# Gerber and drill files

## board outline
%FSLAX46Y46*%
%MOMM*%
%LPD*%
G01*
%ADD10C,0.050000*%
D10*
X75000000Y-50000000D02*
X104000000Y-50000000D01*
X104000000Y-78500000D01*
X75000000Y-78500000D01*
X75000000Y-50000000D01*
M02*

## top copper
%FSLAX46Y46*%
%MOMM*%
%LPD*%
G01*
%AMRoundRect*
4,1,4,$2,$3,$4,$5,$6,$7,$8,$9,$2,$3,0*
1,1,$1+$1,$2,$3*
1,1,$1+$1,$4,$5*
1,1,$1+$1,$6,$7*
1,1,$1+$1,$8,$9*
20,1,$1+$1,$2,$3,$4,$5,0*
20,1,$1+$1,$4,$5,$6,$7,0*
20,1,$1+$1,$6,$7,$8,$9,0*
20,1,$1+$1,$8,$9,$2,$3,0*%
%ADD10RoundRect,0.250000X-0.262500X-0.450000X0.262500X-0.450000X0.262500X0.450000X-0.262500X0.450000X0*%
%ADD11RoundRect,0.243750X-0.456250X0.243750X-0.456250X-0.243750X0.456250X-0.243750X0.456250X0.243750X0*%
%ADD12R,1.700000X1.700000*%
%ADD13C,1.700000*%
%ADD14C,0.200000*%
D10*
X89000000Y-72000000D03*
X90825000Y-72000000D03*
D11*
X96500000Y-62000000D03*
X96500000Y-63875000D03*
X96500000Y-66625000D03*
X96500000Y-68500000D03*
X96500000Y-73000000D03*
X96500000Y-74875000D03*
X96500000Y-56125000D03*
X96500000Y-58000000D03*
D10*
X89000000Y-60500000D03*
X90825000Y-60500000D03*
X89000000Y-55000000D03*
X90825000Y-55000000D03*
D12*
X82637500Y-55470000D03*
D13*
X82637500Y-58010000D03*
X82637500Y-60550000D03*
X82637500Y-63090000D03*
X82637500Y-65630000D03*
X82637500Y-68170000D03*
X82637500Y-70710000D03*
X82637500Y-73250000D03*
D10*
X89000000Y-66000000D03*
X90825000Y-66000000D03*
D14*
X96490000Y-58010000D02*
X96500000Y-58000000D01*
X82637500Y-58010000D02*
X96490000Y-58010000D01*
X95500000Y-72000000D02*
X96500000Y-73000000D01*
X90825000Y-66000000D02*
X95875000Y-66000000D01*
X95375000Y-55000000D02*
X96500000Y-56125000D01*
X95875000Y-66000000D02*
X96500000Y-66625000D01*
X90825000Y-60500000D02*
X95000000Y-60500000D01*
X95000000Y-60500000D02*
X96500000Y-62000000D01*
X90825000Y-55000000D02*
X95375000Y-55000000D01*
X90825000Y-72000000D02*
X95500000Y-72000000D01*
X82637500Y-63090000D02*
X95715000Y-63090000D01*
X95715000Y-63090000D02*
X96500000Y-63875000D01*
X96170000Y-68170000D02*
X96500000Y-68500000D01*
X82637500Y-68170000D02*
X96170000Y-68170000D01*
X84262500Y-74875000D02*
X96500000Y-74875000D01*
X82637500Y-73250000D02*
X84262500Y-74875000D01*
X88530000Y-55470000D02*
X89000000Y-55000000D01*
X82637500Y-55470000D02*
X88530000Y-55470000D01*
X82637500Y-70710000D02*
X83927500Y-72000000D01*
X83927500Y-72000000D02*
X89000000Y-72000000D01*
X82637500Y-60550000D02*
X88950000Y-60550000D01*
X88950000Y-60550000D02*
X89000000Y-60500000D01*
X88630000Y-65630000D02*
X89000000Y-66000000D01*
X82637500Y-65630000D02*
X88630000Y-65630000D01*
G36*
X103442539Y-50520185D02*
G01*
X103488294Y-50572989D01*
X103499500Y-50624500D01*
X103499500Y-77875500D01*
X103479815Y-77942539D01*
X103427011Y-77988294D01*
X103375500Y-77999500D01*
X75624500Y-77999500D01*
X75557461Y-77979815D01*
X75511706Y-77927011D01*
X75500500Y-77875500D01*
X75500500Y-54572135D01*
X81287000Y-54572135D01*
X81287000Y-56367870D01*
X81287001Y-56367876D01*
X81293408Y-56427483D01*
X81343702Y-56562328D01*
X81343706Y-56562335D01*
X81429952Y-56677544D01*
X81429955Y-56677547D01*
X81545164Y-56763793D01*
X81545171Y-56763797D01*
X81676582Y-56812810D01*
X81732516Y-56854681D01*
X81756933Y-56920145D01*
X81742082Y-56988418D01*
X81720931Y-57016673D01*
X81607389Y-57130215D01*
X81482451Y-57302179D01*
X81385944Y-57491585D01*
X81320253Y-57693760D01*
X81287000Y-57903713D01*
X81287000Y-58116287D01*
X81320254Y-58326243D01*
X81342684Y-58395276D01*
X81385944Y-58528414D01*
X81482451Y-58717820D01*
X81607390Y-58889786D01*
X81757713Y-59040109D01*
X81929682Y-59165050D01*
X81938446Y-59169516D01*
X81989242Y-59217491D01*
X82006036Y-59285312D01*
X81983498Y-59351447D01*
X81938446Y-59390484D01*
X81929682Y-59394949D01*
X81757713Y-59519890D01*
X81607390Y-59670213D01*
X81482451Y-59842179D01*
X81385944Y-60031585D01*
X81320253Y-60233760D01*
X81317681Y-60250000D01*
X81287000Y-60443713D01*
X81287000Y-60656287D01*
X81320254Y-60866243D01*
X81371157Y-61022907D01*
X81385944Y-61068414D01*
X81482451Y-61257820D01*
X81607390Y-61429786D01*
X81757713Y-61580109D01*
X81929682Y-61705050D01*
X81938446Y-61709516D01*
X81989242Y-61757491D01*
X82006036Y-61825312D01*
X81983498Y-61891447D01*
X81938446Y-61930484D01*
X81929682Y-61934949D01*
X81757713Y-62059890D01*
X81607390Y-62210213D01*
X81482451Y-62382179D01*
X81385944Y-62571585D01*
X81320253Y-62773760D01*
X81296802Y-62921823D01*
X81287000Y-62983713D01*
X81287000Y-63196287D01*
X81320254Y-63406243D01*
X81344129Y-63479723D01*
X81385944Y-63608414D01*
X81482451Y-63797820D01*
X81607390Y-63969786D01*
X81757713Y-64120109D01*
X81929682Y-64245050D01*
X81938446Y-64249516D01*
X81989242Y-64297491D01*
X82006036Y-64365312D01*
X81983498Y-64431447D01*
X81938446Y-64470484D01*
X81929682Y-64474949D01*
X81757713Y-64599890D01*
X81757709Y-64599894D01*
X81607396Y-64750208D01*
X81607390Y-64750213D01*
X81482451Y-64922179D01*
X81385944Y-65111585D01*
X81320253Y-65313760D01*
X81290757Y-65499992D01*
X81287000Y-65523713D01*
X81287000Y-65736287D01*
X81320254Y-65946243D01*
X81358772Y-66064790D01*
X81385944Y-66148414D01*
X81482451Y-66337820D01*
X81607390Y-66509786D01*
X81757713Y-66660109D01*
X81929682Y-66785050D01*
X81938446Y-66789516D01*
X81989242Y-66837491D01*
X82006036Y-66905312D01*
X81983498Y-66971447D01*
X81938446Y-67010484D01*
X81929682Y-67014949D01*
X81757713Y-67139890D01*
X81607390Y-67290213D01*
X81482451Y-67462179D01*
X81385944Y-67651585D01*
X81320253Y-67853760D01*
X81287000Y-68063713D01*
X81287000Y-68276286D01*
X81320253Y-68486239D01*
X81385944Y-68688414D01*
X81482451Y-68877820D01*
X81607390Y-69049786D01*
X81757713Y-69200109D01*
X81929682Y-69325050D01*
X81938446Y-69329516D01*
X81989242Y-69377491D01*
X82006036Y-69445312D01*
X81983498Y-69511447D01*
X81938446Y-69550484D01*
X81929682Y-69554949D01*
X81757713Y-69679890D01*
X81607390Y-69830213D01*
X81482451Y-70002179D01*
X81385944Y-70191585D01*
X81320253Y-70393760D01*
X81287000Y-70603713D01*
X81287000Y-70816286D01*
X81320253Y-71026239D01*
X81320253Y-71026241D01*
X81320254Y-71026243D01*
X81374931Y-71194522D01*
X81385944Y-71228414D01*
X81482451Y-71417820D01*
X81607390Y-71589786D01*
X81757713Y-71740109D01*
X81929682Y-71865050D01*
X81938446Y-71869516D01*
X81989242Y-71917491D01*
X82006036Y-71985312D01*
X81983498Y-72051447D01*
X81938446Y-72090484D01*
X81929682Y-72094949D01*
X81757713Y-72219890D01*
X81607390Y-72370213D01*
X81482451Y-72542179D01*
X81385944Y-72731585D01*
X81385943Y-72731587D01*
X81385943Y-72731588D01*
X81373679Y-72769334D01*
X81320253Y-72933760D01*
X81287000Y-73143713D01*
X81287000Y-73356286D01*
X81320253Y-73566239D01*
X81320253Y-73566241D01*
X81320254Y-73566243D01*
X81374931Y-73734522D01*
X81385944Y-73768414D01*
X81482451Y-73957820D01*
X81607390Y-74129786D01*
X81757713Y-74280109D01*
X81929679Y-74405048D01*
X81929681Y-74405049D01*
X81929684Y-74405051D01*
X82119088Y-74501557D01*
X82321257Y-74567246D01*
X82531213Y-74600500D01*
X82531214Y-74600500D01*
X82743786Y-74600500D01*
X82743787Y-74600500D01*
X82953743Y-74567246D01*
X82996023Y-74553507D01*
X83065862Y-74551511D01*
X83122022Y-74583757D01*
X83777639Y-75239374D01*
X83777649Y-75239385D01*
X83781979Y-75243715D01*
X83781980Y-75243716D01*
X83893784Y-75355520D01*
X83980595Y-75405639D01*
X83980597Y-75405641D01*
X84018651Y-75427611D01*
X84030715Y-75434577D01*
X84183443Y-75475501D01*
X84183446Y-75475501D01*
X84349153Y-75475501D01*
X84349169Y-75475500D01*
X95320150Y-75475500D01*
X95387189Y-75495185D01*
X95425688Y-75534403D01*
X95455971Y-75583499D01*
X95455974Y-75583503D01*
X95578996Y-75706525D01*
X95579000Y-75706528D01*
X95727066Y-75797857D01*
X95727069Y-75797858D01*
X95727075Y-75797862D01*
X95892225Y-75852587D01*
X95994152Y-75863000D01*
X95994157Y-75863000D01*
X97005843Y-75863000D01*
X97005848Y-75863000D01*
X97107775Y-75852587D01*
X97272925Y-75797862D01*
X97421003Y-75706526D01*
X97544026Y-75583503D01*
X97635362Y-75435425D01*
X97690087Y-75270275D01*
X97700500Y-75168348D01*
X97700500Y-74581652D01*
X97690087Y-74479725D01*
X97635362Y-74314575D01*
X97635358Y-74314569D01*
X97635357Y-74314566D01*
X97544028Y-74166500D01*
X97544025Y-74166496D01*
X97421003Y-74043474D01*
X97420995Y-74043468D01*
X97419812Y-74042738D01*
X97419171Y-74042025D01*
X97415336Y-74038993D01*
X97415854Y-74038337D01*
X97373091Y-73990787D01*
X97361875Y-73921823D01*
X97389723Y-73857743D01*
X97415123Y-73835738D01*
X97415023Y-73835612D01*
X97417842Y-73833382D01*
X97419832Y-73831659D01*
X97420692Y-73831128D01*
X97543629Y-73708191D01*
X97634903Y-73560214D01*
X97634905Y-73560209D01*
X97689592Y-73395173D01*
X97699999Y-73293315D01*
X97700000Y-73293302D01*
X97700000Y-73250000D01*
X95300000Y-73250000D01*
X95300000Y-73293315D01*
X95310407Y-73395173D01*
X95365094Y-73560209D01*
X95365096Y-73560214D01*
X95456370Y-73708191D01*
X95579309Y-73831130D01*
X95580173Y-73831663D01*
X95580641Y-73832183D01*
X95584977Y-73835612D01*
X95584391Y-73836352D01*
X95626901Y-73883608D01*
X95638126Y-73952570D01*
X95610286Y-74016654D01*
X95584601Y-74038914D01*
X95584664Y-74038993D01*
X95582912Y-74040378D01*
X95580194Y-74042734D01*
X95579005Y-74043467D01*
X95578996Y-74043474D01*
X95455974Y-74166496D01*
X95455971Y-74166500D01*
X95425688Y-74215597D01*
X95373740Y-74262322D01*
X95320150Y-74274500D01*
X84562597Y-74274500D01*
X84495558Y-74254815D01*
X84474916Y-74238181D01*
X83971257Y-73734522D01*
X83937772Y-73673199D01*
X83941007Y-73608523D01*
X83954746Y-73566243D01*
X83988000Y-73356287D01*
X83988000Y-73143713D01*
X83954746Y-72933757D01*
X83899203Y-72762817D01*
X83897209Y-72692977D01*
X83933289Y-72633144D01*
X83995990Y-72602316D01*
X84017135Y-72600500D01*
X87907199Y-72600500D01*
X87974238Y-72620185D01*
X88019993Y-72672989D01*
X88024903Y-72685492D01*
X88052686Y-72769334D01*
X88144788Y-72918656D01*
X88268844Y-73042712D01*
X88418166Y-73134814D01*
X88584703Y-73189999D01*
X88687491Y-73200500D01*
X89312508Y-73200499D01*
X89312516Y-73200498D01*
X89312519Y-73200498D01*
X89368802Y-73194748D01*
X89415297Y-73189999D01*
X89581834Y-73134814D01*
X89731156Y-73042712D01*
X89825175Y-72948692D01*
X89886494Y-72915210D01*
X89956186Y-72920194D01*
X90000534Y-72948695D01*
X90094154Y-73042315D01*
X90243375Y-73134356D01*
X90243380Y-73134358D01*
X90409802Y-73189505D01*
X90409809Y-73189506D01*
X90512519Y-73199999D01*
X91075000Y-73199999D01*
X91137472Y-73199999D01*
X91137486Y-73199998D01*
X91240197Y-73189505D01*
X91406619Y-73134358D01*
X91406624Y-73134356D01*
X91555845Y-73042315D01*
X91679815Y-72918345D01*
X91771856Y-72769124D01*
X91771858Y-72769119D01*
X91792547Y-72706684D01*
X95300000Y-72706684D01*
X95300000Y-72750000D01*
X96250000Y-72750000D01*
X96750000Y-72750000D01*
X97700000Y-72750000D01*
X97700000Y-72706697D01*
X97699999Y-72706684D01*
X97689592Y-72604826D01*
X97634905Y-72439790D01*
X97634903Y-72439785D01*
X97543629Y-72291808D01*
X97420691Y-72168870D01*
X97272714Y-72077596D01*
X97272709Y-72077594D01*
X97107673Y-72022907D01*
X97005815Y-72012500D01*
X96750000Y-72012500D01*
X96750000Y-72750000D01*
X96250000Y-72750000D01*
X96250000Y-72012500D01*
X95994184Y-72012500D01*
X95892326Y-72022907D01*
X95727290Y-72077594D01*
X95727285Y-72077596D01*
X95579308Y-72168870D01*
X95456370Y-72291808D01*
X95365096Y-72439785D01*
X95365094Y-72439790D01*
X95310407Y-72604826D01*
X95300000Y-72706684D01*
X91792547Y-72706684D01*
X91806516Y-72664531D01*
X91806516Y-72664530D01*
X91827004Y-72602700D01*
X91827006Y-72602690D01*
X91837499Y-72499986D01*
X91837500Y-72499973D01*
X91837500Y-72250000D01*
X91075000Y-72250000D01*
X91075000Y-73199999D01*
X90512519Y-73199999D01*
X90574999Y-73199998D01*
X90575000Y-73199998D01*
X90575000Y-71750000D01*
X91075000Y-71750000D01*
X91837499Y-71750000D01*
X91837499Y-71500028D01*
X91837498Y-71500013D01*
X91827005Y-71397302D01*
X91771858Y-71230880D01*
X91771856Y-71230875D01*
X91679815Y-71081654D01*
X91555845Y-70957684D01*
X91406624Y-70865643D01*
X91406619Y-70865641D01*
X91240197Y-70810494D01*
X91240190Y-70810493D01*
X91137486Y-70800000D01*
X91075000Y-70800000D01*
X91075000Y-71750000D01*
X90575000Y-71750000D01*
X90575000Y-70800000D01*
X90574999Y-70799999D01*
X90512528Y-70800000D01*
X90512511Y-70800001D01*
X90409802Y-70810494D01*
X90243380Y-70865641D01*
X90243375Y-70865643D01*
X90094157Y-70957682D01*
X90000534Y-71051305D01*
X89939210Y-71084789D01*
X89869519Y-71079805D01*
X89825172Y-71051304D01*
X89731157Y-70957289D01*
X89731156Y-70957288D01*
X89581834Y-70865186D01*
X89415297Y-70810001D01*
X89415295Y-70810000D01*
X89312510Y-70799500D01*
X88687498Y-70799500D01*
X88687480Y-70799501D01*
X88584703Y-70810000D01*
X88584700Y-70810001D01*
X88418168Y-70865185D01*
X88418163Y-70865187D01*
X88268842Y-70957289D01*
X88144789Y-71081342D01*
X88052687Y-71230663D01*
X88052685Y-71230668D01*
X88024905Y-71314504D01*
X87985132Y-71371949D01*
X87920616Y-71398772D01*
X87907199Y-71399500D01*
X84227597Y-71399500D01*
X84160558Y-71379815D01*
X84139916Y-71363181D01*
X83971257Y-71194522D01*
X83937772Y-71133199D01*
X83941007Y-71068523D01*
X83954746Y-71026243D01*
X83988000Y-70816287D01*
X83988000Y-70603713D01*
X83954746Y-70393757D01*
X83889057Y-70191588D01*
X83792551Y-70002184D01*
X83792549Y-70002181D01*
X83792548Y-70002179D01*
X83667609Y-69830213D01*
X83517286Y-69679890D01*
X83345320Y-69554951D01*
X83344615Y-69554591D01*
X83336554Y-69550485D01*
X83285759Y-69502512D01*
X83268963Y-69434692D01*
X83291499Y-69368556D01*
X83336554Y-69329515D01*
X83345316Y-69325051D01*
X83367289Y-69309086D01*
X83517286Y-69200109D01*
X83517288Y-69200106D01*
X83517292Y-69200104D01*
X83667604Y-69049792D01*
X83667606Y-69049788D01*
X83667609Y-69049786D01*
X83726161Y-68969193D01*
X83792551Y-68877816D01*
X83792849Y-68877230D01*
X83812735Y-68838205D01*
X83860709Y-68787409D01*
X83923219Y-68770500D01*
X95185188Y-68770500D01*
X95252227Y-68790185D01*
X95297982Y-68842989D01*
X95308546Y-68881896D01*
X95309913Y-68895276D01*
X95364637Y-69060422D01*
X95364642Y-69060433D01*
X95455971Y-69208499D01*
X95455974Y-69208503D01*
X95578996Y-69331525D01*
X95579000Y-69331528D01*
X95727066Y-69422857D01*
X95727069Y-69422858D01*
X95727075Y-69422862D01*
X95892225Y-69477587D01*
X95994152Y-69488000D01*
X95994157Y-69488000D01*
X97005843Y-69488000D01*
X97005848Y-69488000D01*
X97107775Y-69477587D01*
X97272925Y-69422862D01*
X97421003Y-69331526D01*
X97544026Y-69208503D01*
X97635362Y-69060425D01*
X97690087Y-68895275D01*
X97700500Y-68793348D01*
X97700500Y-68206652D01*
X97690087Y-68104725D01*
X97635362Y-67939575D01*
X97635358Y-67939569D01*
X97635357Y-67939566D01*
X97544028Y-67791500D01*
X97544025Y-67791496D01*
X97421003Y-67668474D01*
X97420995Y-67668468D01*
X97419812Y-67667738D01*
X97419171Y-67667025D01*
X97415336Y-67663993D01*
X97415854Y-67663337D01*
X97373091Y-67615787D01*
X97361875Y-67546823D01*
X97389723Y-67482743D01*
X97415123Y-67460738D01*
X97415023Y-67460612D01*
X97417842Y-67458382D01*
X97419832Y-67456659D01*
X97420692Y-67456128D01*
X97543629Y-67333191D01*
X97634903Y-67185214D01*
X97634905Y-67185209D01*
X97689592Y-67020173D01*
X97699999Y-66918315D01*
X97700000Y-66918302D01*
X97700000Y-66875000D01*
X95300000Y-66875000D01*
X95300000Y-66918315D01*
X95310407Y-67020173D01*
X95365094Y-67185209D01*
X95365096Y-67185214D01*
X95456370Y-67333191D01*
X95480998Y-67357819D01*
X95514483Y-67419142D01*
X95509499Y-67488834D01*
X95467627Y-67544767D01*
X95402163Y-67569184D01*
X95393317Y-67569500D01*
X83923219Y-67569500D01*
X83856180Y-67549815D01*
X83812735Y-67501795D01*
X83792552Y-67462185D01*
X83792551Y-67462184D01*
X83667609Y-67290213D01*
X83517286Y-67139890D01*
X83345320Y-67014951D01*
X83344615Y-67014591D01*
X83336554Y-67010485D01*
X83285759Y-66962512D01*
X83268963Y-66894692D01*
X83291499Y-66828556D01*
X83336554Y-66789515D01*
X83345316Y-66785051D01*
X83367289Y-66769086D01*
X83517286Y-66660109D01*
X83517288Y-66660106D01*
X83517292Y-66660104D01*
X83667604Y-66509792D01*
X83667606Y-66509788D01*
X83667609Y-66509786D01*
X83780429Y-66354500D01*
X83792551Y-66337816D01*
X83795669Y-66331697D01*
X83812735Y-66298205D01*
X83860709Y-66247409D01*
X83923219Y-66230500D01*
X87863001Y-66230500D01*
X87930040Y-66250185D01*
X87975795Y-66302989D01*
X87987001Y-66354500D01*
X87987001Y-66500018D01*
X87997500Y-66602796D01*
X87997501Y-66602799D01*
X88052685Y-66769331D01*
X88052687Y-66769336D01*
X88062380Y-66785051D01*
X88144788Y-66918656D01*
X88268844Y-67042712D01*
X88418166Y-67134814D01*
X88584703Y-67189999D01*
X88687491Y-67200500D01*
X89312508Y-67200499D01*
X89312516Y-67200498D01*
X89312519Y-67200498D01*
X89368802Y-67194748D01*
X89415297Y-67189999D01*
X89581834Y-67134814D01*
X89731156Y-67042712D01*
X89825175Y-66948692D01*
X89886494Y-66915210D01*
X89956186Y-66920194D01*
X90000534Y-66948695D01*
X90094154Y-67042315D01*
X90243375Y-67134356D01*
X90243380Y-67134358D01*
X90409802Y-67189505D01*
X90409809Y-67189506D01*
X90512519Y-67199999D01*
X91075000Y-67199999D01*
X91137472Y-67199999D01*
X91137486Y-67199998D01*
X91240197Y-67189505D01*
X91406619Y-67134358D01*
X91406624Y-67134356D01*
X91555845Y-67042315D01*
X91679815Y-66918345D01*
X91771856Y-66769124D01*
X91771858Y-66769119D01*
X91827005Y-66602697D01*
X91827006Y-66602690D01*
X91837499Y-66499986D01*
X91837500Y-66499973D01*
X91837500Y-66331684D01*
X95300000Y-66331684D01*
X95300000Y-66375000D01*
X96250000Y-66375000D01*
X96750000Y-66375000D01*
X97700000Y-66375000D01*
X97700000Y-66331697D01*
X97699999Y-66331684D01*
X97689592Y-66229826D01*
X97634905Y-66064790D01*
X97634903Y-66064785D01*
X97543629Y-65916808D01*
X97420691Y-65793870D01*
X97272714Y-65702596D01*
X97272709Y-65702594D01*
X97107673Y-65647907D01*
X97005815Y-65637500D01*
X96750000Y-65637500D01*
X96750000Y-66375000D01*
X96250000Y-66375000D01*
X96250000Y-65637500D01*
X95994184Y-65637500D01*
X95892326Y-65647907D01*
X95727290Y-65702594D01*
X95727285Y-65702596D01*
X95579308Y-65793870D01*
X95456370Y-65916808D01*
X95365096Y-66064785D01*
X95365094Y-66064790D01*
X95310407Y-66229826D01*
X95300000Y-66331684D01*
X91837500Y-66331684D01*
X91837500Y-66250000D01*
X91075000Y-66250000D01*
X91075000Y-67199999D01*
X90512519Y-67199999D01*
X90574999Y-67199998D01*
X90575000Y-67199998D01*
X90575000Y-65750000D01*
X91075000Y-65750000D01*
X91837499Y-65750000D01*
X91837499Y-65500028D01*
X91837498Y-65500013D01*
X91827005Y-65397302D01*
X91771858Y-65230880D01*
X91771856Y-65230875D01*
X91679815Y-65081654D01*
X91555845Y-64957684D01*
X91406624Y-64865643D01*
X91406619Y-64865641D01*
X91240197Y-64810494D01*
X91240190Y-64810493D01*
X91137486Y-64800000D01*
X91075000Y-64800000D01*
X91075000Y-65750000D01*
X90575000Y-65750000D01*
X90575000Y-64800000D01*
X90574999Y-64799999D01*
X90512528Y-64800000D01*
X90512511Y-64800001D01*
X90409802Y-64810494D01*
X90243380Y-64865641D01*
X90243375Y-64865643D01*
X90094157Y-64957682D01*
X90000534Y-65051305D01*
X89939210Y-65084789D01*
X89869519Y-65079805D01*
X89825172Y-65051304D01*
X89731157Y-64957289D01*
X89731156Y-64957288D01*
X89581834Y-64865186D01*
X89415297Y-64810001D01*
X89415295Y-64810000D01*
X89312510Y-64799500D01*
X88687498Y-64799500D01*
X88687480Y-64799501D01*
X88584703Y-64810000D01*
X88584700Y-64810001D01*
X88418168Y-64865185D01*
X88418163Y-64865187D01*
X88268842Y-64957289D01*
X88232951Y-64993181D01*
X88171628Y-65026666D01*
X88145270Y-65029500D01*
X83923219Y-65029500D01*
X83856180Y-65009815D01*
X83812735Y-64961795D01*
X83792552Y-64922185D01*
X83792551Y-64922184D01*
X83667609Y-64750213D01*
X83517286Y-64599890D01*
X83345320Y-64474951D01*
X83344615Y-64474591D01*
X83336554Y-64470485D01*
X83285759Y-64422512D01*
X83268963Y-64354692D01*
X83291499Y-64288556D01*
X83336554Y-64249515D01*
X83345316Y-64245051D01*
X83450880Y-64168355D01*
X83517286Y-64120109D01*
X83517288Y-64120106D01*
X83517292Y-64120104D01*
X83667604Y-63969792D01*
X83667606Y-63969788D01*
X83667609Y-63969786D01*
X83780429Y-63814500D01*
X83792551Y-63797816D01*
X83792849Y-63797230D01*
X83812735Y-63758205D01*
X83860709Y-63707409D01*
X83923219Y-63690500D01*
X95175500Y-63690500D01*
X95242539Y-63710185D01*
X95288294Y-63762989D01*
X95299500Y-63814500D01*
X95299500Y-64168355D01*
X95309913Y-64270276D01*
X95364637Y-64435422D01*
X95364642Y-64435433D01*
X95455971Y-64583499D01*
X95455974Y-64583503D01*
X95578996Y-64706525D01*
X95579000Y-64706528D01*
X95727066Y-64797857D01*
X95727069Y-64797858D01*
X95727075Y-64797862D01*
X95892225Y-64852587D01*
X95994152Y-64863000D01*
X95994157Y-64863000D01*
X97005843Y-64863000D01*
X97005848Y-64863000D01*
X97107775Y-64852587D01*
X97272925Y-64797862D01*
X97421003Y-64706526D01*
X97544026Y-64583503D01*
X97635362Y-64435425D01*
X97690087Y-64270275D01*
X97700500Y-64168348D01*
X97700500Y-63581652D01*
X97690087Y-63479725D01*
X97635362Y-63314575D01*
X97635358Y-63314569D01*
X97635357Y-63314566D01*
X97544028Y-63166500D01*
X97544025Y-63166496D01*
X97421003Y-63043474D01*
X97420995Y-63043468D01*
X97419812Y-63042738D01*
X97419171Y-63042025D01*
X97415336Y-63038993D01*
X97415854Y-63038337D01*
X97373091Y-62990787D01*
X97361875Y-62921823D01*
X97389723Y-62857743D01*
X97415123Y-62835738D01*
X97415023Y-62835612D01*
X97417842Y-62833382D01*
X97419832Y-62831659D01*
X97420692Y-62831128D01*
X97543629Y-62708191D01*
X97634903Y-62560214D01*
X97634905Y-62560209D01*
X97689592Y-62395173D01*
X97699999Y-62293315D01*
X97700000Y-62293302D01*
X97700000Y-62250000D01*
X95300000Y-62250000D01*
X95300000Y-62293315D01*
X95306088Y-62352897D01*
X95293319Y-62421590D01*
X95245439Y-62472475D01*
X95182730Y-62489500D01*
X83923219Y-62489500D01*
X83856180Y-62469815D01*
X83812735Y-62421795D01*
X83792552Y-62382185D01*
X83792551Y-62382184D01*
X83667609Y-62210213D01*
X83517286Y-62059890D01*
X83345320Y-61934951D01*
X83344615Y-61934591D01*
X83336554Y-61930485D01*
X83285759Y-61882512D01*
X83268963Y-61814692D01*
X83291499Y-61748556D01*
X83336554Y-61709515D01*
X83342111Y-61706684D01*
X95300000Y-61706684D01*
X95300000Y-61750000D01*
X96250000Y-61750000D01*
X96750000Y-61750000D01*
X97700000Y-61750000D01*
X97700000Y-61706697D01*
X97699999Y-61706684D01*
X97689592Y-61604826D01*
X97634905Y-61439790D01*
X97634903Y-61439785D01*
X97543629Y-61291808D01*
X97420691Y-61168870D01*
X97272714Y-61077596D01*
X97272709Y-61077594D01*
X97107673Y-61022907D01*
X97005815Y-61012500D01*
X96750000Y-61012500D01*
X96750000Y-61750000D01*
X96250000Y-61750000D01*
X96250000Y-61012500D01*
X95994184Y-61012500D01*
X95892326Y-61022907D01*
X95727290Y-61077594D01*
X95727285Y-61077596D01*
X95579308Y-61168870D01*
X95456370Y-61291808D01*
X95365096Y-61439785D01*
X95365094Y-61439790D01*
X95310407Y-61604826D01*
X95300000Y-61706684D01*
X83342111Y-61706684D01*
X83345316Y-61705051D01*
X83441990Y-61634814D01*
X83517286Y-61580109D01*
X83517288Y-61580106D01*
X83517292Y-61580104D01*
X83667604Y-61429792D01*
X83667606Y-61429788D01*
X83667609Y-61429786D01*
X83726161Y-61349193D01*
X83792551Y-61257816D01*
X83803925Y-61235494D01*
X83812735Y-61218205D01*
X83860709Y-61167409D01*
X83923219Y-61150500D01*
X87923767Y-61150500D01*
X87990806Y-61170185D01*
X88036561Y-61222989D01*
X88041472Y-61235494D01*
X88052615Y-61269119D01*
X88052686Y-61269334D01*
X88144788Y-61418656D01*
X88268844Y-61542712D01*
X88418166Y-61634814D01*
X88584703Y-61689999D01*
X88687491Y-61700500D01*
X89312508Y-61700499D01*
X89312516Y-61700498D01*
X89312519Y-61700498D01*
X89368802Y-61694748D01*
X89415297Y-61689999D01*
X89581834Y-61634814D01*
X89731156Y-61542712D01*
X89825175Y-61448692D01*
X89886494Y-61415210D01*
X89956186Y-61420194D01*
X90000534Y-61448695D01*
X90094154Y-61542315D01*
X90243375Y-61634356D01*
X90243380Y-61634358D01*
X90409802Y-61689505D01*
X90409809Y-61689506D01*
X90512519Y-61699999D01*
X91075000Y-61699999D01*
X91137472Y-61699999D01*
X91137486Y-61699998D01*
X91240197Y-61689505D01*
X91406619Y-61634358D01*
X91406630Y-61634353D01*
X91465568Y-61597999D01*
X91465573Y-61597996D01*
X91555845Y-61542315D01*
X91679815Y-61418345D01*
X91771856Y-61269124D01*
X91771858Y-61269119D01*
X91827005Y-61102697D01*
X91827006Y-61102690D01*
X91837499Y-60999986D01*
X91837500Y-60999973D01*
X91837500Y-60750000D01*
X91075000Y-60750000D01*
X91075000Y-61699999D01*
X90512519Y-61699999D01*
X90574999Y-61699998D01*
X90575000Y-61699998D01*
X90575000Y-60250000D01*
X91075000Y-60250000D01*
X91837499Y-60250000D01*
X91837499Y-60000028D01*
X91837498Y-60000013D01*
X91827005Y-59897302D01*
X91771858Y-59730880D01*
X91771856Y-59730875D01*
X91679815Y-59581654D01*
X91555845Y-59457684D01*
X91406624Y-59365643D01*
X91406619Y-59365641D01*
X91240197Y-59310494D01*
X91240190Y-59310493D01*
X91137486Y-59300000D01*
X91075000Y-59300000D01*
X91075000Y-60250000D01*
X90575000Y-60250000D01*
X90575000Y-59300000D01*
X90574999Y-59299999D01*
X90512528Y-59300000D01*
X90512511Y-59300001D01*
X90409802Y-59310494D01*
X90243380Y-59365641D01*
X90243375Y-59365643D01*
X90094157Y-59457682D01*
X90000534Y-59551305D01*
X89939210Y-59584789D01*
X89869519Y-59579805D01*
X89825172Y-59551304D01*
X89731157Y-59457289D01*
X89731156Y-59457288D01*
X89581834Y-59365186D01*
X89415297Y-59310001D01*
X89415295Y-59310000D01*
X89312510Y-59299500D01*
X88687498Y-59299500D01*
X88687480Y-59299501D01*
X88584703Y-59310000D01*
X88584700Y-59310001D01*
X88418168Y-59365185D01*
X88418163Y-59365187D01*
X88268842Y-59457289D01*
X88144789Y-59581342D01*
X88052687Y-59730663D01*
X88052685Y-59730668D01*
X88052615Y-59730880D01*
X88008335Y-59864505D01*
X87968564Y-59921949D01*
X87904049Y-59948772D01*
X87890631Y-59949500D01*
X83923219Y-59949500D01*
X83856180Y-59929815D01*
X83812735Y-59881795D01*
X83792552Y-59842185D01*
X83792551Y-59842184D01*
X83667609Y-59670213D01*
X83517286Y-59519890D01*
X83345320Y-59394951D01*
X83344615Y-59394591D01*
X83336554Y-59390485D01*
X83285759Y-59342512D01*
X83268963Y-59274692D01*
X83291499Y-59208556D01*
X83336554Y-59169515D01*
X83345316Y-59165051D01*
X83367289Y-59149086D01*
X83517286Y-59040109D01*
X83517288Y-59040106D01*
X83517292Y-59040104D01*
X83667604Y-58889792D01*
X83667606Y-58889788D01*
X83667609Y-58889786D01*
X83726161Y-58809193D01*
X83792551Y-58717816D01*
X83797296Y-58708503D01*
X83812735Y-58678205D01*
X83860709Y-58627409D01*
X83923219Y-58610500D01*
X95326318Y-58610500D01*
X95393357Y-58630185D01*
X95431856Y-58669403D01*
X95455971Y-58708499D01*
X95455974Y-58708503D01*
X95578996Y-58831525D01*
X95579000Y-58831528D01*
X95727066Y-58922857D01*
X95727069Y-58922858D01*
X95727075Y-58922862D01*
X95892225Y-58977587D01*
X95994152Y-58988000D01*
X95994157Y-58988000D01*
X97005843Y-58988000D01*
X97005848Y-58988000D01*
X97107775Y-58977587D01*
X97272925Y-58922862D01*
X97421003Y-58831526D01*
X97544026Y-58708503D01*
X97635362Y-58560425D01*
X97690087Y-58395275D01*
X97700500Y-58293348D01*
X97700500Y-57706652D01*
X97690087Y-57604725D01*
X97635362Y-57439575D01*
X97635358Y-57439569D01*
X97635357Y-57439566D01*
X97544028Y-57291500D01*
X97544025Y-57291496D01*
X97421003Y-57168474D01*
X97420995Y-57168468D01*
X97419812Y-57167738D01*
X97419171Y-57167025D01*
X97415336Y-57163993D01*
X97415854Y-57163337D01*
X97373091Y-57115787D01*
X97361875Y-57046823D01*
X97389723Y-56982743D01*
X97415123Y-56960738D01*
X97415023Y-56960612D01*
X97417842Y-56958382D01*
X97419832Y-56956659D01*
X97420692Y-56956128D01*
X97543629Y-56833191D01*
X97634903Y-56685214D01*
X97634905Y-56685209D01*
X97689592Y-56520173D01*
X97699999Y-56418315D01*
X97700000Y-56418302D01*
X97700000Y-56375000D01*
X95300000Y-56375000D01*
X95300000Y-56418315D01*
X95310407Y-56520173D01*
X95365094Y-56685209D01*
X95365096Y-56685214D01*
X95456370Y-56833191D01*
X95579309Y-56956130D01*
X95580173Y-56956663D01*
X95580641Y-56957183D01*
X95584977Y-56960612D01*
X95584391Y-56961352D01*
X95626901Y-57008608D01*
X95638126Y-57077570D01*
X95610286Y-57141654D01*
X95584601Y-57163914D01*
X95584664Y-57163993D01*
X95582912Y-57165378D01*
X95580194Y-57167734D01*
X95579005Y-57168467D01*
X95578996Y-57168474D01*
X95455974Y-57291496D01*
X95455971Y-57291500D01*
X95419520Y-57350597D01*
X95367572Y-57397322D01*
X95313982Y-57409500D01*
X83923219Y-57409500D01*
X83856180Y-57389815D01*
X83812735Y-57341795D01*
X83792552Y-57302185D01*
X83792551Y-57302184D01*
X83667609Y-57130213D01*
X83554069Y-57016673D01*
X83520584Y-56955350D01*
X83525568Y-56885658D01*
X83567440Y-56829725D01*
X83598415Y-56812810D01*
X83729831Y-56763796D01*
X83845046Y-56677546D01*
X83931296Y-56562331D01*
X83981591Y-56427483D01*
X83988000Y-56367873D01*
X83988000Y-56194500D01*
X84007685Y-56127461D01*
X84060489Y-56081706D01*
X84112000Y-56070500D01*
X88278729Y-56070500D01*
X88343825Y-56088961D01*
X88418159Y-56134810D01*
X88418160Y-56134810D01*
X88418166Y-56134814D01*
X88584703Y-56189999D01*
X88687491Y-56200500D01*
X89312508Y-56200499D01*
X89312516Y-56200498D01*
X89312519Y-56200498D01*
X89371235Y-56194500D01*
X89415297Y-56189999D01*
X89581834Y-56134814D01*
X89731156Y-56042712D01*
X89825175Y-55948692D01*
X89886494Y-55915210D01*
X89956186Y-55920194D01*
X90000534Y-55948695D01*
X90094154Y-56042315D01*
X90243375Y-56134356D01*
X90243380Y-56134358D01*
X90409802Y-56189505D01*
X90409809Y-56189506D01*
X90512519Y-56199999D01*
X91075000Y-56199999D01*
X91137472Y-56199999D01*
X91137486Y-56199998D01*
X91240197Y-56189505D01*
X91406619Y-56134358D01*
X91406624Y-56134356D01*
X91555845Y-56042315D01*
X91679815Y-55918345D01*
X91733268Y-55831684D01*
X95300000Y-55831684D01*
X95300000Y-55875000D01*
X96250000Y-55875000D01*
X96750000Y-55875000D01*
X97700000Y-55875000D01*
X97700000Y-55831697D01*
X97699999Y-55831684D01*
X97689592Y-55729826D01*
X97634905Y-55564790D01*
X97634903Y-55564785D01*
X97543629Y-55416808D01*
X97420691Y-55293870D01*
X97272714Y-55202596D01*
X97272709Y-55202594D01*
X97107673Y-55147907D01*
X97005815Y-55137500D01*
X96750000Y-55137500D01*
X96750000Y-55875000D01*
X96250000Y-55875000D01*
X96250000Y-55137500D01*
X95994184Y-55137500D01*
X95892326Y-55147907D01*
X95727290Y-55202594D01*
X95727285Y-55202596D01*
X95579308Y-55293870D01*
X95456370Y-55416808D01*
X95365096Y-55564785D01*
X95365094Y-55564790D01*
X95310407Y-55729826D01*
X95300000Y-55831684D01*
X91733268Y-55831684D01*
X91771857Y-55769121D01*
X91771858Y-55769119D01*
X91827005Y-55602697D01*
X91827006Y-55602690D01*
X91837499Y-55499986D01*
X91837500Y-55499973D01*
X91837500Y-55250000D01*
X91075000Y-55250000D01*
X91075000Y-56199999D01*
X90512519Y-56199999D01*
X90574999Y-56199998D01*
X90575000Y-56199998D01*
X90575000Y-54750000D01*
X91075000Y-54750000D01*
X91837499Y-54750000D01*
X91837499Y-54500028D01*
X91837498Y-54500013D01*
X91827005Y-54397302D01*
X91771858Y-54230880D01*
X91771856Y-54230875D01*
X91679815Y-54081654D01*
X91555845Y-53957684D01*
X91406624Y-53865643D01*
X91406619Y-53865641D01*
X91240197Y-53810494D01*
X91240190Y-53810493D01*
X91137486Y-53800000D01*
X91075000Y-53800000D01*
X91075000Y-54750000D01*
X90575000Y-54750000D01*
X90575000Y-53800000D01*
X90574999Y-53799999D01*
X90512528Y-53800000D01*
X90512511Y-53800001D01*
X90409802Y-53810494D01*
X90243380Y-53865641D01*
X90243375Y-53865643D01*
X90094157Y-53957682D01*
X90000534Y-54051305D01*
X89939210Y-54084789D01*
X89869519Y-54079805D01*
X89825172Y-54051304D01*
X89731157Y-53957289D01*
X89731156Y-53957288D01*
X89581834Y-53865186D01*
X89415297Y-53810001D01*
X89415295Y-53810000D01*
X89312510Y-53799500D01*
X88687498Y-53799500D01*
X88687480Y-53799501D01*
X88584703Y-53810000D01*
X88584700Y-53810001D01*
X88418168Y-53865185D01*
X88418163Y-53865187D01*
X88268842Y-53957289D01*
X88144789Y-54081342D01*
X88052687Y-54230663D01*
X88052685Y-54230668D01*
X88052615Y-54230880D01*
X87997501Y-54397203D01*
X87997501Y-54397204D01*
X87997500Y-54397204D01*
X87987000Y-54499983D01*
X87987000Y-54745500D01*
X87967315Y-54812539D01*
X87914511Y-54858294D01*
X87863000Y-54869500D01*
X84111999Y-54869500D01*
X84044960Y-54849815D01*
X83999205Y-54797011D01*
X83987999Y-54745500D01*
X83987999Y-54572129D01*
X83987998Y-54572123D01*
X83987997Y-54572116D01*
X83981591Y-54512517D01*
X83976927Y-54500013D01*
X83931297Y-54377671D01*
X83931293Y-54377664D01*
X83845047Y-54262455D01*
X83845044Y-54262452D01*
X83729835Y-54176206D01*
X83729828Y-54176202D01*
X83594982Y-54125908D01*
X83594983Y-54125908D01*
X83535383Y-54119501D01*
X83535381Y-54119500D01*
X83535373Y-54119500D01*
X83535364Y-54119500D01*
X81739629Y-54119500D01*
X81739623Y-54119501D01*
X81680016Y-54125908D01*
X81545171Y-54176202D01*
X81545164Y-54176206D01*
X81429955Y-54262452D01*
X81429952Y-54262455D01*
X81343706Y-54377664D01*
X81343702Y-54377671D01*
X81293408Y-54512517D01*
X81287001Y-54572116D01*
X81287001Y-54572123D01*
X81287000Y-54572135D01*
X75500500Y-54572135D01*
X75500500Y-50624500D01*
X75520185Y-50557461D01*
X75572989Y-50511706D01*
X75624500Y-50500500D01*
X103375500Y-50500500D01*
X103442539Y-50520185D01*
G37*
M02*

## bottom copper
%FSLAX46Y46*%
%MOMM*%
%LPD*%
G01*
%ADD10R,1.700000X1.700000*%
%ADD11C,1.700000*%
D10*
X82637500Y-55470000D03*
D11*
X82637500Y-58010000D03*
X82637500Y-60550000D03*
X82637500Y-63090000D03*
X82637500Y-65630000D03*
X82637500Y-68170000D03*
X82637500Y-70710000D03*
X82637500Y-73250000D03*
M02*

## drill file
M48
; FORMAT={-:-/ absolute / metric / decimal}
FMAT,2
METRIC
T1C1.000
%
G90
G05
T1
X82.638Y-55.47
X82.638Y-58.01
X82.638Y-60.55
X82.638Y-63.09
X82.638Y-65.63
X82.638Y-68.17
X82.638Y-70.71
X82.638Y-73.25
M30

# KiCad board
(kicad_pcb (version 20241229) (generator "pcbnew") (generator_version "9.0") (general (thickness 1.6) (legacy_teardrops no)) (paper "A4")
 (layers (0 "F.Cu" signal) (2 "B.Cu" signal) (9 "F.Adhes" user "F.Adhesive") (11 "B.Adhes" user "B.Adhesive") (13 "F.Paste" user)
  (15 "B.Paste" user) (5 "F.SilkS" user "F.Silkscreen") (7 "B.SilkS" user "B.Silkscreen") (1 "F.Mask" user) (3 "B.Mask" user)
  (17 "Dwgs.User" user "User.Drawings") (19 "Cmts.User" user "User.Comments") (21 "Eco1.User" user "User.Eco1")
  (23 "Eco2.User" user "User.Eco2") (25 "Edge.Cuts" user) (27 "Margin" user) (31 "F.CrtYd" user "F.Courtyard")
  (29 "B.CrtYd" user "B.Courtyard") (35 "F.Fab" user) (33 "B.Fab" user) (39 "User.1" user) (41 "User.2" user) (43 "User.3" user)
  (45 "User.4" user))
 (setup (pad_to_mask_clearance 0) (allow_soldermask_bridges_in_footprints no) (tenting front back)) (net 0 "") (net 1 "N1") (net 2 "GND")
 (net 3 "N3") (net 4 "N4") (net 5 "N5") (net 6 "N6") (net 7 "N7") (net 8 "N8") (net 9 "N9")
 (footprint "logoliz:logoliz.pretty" (layer "F.Cu") (at 101 53.5)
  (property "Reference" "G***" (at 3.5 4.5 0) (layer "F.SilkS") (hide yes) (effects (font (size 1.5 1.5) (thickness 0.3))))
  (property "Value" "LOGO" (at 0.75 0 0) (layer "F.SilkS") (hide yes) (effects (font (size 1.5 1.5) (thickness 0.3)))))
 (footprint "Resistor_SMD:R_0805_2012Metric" (layer "F.Cu") (at 89.9125 72)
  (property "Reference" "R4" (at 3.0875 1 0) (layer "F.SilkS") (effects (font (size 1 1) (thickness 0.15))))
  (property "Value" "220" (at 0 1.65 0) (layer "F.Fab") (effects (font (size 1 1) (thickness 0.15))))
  (pad "1" smd roundrect (at -0.9125 0) (size 1.025 1.4) (layers "F.Cu" "F.Mask" "F.Paste") (roundrect_rratio 0.243902) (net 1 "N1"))
  (pad "2" smd roundrect (at 0.9125 0) (size 1.025 1.4) (layers "F.Cu" "F.Mask" "F.Paste") (roundrect_rratio 0.243902) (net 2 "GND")))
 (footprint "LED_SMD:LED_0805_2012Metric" (layer "F.Cu") (at 96.5 62.9375 -90)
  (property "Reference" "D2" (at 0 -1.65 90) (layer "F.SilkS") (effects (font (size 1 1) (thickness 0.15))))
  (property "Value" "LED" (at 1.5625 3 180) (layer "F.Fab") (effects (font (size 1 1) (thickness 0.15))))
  (pad "1" smd roundrect (at -0.9375 0 270) (size 0.975 1.4) (layers "F.Cu" "F.Mask" "F.Paste") (roundrect_rratio 0.25) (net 2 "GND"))
  (pad "2" smd roundrect (at 0.9375 0 270) (size 0.975 1.4) (layers "F.Cu" "F.Mask" "F.Paste") (roundrect_rratio 0.25) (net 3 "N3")))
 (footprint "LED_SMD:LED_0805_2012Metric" (layer "F.Cu") (at 96.5 67.5625 -90)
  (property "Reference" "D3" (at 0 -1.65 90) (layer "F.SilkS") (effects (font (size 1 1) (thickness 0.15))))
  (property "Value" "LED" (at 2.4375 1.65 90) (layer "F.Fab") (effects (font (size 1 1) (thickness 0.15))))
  (pad "1" smd roundrect (at -0.9375 0 270) (size 0.975 1.4) (layers "F.Cu" "F.Mask" "F.Paste") (roundrect_rratio 0.25) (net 2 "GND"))
  (pad "2" smd roundrect (at 0.9375 0 270) (size 0.975 1.4) (layers "F.Cu" "F.Mask" "F.Paste") (roundrect_rratio 0.25) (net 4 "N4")))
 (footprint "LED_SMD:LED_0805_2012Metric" (layer "F.Cu") (at 96.5 73.9375 -90)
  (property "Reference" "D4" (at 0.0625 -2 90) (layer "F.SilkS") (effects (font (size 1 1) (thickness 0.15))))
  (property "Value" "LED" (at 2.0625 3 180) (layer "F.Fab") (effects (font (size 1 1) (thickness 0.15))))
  (pad "1" smd roundrect (at -0.9375 0 270) (size 0.975 1.4) (layers "F.Cu" "F.Mask" "F.Paste") (roundrect_rratio 0.25) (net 2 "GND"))
  (pad "2" smd roundrect (at 0.9375 0 270) (size 0.975 1.4) (layers "F.Cu" "F.Mask" "F.Paste") (roundrect_rratio 0.25) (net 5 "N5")))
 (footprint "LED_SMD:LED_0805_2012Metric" (layer "F.Cu") (at 96.5 57.0625 -90)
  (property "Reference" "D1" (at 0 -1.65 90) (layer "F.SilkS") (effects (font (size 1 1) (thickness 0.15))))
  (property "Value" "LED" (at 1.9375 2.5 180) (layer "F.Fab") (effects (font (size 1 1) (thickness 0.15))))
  (pad "1" smd roundrect (at -0.9375 0 270) (size 0.975 1.4) (layers "F.Cu" "F.Mask" "F.Paste") (roundrect_rratio 0.25) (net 2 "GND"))
  (pad "2" smd roundrect (at 0.9375 0 270) (size 0.975 1.4) (layers "F.Cu" "F.Mask" "F.Paste") (roundrect_rratio 0.25) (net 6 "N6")))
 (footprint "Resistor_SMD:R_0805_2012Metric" (layer "F.Cu") (at 89.9125 60.5)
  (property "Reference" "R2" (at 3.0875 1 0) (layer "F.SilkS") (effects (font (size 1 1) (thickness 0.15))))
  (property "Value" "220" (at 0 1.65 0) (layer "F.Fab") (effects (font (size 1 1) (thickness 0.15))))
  (pad "1" smd roundrect (at -0.9125 0) (size 1.025 1.4) (layers "F.Cu" "F.Mask" "F.Paste") (roundrect_rratio 0.243902) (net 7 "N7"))
  (pad "2" smd roundrect (at 0.9125 0) (size 1.025 1.4) (layers "F.Cu" "F.Mask" "F.Paste") (roundrect_rratio 0.243902) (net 2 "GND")))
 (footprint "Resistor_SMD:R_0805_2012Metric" (layer "F.Cu") (at 89.9125 55)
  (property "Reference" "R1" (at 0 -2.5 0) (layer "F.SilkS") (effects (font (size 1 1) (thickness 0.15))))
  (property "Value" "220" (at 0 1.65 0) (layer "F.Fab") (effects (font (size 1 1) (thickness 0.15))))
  (pad "1" smd roundrect (at -0.9125 0) (size 1.025 1.4) (layers "F.Cu" "F.Mask" "F.Paste") (roundrect_rratio 0.243902) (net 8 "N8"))
  (pad "2" smd roundrect (at 0.9125 0) (size 1.025 1.4) (layers "F.Cu" "F.Mask" "F.Paste") (roundrect_rratio 0.243902) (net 2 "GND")))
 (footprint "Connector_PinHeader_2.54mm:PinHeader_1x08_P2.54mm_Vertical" (layer "F.Cu") (at 82.6375 55.47)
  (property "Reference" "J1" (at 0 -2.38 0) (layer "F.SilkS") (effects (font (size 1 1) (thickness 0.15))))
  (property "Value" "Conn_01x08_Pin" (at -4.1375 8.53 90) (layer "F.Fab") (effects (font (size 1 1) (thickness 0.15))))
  (pad "1" thru_hole rect (at 0 0) (size 1.7 1.7) (drill 1) (layers "*.Cu" "*.Mask") (remove_unused_layers no) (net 8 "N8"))
  (pad "2" thru_hole circle (at 0 2.54) (size 1.7 1.7) (drill 1) (layers "*.Cu" "*.Mask") (remove_unused_layers no) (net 6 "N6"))
  (pad "3" thru_hole circle (at 0 5.08) (size 1.7 1.7) (drill 1) (layers "*.Cu" "*.Mask") (remove_unused_layers no) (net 7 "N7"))
  (pad "4" thru_hole circle (at 0 7.62) (size 1.7 1.7) (drill 1) (layers "*.Cu" "*.Mask") (remove_unused_layers no) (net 3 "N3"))
  (pad "5" thru_hole circle (at 0 10.16) (size 1.7 1.7) (drill 1) (layers "*.Cu" "*.Mask") (remove_unused_layers no) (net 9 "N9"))
  (pad "6" thru_hole circle (at 0 12.7) (size 1.7 1.7) (drill 1) (layers "*.Cu" "*.Mask") (remove_unused_layers no) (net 4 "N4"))
  (pad "7" thru_hole circle (at 0 15.24) (size 1.7 1.7) (drill 1) (layers "*.Cu" "*.Mask") (remove_unused_layers no) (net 1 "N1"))
  (pad "8" thru_hole circle (at 0 17.78) (size 1.7 1.7) (drill 1) (layers "*.Cu" "*.Mask") (remove_unused_layers no) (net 5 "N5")))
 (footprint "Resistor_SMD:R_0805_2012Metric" (layer "F.Cu") (at 89.9125 66)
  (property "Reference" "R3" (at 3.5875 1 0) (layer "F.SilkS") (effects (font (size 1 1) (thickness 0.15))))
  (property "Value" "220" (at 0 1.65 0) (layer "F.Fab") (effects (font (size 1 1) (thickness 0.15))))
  (pad "1" smd roundrect (at -0.9125 0) (size 1.025 1.4) (layers "F.Cu" "F.Mask" "F.Paste") (roundrect_rratio 0.243902) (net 9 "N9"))
  (pad "2" smd roundrect (at 0.9125 0) (size 1.025 1.4) (layers "F.Cu" "F.Mask" "F.Paste") (roundrect_rratio 0.243902) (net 2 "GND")))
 (gr_rect (start 75 50) (end 104 78.5) (stroke (width 0.05) (type default)) (fill no) (layer "Edge.Cuts"))
 (segment (start 96.49 58.01) (end 96.5 58) (width 0.2) (layer "F.Cu") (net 6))
 (segment (start 82.6375 58.01) (end 96.49 58.01) (width 0.2) (layer "F.Cu") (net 6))
 (segment (start 95.5 72) (end 96.5 73) (width 0.2) (layer "F.Cu") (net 2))
 (segment (start 90.825 66) (end 95.875 66) (width 0.2) (layer "F.Cu") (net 2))
 (segment (start 95.375 55) (end 96.5 56.125) (width 0.2) (layer "F.Cu") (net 2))
 (segment (start 95.875 66) (end 96.5 66.625) (width 0.2) (layer "F.Cu") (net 2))
 (segment (start 90.825 60.5) (end 95 60.5) (width 0.2) (layer "F.Cu") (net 2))
 (segment (start 95 60.5) (end 96.5 62) (width 0.2) (layer "F.Cu") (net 2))
 (segment (start 90.825 55) (end 95.375 55) (width 0.2) (layer "F.Cu") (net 2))
 (segment (start 90.825 72) (end 95.5 72) (width 0.2) (layer "F.Cu") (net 2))
 (segment (start 82.6375 63.09) (end 95.715 63.09) (width 0.2) (layer "F.Cu") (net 3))
 (segment (start 95.715 63.09) (end 96.5 63.875) (width 0.2) (layer "F.Cu") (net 3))
 (segment (start 96.17 68.17) (end 96.5 68.5) (width 0.2) (layer "F.Cu") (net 4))
 (segment (start 82.6375 68.17) (end 96.17 68.17) (width 0.2) (layer "F.Cu") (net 4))
 (segment (start 84.2625 74.875) (end 96.5 74.875) (width 0.2) (layer "F.Cu") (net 5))
 (segment (start 82.6375 73.25) (end 84.2625 74.875) (width 0.2) (layer "F.Cu") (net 5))
 (segment (start 88.53 55.47) (end 89 55) (width 0.2) (layer "F.Cu") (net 8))
 (segment (start 82.6375 55.47) (end 88.53 55.47) (width 0.2) (layer "F.Cu") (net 8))
 (segment (start 82.6375 70.71) (end 83.9275 72) (width 0.2) (layer "F.Cu") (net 1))
 (segment (start 83.9275 72) (end 89 72) (width 0.2) (layer "F.Cu") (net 1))
 (segment (start 82.6375 60.55) (end 88.95 60.55) (width 0.2) (layer "F.Cu") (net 7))
 (segment (start 88.95 60.55) (end 89 60.5) (width 0.2) (layer "F.Cu") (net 7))
 (segment (start 88.63 65.63) (end 89 66) (width 0.2) (layer "F.Cu") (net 9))
 (segment (start 82.6375 65.63) (end 88.63 65.63) (width 0.2) (layer "F.Cu") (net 9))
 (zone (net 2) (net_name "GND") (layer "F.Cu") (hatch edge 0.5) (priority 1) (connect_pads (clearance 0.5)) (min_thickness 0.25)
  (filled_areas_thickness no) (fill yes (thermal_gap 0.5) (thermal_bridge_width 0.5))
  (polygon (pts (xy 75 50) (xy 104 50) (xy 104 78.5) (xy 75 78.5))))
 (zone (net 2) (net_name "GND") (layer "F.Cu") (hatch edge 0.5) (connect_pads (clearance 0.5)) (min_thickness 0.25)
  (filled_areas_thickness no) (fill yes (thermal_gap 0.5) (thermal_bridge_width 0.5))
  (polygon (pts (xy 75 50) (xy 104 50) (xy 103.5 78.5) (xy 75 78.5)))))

